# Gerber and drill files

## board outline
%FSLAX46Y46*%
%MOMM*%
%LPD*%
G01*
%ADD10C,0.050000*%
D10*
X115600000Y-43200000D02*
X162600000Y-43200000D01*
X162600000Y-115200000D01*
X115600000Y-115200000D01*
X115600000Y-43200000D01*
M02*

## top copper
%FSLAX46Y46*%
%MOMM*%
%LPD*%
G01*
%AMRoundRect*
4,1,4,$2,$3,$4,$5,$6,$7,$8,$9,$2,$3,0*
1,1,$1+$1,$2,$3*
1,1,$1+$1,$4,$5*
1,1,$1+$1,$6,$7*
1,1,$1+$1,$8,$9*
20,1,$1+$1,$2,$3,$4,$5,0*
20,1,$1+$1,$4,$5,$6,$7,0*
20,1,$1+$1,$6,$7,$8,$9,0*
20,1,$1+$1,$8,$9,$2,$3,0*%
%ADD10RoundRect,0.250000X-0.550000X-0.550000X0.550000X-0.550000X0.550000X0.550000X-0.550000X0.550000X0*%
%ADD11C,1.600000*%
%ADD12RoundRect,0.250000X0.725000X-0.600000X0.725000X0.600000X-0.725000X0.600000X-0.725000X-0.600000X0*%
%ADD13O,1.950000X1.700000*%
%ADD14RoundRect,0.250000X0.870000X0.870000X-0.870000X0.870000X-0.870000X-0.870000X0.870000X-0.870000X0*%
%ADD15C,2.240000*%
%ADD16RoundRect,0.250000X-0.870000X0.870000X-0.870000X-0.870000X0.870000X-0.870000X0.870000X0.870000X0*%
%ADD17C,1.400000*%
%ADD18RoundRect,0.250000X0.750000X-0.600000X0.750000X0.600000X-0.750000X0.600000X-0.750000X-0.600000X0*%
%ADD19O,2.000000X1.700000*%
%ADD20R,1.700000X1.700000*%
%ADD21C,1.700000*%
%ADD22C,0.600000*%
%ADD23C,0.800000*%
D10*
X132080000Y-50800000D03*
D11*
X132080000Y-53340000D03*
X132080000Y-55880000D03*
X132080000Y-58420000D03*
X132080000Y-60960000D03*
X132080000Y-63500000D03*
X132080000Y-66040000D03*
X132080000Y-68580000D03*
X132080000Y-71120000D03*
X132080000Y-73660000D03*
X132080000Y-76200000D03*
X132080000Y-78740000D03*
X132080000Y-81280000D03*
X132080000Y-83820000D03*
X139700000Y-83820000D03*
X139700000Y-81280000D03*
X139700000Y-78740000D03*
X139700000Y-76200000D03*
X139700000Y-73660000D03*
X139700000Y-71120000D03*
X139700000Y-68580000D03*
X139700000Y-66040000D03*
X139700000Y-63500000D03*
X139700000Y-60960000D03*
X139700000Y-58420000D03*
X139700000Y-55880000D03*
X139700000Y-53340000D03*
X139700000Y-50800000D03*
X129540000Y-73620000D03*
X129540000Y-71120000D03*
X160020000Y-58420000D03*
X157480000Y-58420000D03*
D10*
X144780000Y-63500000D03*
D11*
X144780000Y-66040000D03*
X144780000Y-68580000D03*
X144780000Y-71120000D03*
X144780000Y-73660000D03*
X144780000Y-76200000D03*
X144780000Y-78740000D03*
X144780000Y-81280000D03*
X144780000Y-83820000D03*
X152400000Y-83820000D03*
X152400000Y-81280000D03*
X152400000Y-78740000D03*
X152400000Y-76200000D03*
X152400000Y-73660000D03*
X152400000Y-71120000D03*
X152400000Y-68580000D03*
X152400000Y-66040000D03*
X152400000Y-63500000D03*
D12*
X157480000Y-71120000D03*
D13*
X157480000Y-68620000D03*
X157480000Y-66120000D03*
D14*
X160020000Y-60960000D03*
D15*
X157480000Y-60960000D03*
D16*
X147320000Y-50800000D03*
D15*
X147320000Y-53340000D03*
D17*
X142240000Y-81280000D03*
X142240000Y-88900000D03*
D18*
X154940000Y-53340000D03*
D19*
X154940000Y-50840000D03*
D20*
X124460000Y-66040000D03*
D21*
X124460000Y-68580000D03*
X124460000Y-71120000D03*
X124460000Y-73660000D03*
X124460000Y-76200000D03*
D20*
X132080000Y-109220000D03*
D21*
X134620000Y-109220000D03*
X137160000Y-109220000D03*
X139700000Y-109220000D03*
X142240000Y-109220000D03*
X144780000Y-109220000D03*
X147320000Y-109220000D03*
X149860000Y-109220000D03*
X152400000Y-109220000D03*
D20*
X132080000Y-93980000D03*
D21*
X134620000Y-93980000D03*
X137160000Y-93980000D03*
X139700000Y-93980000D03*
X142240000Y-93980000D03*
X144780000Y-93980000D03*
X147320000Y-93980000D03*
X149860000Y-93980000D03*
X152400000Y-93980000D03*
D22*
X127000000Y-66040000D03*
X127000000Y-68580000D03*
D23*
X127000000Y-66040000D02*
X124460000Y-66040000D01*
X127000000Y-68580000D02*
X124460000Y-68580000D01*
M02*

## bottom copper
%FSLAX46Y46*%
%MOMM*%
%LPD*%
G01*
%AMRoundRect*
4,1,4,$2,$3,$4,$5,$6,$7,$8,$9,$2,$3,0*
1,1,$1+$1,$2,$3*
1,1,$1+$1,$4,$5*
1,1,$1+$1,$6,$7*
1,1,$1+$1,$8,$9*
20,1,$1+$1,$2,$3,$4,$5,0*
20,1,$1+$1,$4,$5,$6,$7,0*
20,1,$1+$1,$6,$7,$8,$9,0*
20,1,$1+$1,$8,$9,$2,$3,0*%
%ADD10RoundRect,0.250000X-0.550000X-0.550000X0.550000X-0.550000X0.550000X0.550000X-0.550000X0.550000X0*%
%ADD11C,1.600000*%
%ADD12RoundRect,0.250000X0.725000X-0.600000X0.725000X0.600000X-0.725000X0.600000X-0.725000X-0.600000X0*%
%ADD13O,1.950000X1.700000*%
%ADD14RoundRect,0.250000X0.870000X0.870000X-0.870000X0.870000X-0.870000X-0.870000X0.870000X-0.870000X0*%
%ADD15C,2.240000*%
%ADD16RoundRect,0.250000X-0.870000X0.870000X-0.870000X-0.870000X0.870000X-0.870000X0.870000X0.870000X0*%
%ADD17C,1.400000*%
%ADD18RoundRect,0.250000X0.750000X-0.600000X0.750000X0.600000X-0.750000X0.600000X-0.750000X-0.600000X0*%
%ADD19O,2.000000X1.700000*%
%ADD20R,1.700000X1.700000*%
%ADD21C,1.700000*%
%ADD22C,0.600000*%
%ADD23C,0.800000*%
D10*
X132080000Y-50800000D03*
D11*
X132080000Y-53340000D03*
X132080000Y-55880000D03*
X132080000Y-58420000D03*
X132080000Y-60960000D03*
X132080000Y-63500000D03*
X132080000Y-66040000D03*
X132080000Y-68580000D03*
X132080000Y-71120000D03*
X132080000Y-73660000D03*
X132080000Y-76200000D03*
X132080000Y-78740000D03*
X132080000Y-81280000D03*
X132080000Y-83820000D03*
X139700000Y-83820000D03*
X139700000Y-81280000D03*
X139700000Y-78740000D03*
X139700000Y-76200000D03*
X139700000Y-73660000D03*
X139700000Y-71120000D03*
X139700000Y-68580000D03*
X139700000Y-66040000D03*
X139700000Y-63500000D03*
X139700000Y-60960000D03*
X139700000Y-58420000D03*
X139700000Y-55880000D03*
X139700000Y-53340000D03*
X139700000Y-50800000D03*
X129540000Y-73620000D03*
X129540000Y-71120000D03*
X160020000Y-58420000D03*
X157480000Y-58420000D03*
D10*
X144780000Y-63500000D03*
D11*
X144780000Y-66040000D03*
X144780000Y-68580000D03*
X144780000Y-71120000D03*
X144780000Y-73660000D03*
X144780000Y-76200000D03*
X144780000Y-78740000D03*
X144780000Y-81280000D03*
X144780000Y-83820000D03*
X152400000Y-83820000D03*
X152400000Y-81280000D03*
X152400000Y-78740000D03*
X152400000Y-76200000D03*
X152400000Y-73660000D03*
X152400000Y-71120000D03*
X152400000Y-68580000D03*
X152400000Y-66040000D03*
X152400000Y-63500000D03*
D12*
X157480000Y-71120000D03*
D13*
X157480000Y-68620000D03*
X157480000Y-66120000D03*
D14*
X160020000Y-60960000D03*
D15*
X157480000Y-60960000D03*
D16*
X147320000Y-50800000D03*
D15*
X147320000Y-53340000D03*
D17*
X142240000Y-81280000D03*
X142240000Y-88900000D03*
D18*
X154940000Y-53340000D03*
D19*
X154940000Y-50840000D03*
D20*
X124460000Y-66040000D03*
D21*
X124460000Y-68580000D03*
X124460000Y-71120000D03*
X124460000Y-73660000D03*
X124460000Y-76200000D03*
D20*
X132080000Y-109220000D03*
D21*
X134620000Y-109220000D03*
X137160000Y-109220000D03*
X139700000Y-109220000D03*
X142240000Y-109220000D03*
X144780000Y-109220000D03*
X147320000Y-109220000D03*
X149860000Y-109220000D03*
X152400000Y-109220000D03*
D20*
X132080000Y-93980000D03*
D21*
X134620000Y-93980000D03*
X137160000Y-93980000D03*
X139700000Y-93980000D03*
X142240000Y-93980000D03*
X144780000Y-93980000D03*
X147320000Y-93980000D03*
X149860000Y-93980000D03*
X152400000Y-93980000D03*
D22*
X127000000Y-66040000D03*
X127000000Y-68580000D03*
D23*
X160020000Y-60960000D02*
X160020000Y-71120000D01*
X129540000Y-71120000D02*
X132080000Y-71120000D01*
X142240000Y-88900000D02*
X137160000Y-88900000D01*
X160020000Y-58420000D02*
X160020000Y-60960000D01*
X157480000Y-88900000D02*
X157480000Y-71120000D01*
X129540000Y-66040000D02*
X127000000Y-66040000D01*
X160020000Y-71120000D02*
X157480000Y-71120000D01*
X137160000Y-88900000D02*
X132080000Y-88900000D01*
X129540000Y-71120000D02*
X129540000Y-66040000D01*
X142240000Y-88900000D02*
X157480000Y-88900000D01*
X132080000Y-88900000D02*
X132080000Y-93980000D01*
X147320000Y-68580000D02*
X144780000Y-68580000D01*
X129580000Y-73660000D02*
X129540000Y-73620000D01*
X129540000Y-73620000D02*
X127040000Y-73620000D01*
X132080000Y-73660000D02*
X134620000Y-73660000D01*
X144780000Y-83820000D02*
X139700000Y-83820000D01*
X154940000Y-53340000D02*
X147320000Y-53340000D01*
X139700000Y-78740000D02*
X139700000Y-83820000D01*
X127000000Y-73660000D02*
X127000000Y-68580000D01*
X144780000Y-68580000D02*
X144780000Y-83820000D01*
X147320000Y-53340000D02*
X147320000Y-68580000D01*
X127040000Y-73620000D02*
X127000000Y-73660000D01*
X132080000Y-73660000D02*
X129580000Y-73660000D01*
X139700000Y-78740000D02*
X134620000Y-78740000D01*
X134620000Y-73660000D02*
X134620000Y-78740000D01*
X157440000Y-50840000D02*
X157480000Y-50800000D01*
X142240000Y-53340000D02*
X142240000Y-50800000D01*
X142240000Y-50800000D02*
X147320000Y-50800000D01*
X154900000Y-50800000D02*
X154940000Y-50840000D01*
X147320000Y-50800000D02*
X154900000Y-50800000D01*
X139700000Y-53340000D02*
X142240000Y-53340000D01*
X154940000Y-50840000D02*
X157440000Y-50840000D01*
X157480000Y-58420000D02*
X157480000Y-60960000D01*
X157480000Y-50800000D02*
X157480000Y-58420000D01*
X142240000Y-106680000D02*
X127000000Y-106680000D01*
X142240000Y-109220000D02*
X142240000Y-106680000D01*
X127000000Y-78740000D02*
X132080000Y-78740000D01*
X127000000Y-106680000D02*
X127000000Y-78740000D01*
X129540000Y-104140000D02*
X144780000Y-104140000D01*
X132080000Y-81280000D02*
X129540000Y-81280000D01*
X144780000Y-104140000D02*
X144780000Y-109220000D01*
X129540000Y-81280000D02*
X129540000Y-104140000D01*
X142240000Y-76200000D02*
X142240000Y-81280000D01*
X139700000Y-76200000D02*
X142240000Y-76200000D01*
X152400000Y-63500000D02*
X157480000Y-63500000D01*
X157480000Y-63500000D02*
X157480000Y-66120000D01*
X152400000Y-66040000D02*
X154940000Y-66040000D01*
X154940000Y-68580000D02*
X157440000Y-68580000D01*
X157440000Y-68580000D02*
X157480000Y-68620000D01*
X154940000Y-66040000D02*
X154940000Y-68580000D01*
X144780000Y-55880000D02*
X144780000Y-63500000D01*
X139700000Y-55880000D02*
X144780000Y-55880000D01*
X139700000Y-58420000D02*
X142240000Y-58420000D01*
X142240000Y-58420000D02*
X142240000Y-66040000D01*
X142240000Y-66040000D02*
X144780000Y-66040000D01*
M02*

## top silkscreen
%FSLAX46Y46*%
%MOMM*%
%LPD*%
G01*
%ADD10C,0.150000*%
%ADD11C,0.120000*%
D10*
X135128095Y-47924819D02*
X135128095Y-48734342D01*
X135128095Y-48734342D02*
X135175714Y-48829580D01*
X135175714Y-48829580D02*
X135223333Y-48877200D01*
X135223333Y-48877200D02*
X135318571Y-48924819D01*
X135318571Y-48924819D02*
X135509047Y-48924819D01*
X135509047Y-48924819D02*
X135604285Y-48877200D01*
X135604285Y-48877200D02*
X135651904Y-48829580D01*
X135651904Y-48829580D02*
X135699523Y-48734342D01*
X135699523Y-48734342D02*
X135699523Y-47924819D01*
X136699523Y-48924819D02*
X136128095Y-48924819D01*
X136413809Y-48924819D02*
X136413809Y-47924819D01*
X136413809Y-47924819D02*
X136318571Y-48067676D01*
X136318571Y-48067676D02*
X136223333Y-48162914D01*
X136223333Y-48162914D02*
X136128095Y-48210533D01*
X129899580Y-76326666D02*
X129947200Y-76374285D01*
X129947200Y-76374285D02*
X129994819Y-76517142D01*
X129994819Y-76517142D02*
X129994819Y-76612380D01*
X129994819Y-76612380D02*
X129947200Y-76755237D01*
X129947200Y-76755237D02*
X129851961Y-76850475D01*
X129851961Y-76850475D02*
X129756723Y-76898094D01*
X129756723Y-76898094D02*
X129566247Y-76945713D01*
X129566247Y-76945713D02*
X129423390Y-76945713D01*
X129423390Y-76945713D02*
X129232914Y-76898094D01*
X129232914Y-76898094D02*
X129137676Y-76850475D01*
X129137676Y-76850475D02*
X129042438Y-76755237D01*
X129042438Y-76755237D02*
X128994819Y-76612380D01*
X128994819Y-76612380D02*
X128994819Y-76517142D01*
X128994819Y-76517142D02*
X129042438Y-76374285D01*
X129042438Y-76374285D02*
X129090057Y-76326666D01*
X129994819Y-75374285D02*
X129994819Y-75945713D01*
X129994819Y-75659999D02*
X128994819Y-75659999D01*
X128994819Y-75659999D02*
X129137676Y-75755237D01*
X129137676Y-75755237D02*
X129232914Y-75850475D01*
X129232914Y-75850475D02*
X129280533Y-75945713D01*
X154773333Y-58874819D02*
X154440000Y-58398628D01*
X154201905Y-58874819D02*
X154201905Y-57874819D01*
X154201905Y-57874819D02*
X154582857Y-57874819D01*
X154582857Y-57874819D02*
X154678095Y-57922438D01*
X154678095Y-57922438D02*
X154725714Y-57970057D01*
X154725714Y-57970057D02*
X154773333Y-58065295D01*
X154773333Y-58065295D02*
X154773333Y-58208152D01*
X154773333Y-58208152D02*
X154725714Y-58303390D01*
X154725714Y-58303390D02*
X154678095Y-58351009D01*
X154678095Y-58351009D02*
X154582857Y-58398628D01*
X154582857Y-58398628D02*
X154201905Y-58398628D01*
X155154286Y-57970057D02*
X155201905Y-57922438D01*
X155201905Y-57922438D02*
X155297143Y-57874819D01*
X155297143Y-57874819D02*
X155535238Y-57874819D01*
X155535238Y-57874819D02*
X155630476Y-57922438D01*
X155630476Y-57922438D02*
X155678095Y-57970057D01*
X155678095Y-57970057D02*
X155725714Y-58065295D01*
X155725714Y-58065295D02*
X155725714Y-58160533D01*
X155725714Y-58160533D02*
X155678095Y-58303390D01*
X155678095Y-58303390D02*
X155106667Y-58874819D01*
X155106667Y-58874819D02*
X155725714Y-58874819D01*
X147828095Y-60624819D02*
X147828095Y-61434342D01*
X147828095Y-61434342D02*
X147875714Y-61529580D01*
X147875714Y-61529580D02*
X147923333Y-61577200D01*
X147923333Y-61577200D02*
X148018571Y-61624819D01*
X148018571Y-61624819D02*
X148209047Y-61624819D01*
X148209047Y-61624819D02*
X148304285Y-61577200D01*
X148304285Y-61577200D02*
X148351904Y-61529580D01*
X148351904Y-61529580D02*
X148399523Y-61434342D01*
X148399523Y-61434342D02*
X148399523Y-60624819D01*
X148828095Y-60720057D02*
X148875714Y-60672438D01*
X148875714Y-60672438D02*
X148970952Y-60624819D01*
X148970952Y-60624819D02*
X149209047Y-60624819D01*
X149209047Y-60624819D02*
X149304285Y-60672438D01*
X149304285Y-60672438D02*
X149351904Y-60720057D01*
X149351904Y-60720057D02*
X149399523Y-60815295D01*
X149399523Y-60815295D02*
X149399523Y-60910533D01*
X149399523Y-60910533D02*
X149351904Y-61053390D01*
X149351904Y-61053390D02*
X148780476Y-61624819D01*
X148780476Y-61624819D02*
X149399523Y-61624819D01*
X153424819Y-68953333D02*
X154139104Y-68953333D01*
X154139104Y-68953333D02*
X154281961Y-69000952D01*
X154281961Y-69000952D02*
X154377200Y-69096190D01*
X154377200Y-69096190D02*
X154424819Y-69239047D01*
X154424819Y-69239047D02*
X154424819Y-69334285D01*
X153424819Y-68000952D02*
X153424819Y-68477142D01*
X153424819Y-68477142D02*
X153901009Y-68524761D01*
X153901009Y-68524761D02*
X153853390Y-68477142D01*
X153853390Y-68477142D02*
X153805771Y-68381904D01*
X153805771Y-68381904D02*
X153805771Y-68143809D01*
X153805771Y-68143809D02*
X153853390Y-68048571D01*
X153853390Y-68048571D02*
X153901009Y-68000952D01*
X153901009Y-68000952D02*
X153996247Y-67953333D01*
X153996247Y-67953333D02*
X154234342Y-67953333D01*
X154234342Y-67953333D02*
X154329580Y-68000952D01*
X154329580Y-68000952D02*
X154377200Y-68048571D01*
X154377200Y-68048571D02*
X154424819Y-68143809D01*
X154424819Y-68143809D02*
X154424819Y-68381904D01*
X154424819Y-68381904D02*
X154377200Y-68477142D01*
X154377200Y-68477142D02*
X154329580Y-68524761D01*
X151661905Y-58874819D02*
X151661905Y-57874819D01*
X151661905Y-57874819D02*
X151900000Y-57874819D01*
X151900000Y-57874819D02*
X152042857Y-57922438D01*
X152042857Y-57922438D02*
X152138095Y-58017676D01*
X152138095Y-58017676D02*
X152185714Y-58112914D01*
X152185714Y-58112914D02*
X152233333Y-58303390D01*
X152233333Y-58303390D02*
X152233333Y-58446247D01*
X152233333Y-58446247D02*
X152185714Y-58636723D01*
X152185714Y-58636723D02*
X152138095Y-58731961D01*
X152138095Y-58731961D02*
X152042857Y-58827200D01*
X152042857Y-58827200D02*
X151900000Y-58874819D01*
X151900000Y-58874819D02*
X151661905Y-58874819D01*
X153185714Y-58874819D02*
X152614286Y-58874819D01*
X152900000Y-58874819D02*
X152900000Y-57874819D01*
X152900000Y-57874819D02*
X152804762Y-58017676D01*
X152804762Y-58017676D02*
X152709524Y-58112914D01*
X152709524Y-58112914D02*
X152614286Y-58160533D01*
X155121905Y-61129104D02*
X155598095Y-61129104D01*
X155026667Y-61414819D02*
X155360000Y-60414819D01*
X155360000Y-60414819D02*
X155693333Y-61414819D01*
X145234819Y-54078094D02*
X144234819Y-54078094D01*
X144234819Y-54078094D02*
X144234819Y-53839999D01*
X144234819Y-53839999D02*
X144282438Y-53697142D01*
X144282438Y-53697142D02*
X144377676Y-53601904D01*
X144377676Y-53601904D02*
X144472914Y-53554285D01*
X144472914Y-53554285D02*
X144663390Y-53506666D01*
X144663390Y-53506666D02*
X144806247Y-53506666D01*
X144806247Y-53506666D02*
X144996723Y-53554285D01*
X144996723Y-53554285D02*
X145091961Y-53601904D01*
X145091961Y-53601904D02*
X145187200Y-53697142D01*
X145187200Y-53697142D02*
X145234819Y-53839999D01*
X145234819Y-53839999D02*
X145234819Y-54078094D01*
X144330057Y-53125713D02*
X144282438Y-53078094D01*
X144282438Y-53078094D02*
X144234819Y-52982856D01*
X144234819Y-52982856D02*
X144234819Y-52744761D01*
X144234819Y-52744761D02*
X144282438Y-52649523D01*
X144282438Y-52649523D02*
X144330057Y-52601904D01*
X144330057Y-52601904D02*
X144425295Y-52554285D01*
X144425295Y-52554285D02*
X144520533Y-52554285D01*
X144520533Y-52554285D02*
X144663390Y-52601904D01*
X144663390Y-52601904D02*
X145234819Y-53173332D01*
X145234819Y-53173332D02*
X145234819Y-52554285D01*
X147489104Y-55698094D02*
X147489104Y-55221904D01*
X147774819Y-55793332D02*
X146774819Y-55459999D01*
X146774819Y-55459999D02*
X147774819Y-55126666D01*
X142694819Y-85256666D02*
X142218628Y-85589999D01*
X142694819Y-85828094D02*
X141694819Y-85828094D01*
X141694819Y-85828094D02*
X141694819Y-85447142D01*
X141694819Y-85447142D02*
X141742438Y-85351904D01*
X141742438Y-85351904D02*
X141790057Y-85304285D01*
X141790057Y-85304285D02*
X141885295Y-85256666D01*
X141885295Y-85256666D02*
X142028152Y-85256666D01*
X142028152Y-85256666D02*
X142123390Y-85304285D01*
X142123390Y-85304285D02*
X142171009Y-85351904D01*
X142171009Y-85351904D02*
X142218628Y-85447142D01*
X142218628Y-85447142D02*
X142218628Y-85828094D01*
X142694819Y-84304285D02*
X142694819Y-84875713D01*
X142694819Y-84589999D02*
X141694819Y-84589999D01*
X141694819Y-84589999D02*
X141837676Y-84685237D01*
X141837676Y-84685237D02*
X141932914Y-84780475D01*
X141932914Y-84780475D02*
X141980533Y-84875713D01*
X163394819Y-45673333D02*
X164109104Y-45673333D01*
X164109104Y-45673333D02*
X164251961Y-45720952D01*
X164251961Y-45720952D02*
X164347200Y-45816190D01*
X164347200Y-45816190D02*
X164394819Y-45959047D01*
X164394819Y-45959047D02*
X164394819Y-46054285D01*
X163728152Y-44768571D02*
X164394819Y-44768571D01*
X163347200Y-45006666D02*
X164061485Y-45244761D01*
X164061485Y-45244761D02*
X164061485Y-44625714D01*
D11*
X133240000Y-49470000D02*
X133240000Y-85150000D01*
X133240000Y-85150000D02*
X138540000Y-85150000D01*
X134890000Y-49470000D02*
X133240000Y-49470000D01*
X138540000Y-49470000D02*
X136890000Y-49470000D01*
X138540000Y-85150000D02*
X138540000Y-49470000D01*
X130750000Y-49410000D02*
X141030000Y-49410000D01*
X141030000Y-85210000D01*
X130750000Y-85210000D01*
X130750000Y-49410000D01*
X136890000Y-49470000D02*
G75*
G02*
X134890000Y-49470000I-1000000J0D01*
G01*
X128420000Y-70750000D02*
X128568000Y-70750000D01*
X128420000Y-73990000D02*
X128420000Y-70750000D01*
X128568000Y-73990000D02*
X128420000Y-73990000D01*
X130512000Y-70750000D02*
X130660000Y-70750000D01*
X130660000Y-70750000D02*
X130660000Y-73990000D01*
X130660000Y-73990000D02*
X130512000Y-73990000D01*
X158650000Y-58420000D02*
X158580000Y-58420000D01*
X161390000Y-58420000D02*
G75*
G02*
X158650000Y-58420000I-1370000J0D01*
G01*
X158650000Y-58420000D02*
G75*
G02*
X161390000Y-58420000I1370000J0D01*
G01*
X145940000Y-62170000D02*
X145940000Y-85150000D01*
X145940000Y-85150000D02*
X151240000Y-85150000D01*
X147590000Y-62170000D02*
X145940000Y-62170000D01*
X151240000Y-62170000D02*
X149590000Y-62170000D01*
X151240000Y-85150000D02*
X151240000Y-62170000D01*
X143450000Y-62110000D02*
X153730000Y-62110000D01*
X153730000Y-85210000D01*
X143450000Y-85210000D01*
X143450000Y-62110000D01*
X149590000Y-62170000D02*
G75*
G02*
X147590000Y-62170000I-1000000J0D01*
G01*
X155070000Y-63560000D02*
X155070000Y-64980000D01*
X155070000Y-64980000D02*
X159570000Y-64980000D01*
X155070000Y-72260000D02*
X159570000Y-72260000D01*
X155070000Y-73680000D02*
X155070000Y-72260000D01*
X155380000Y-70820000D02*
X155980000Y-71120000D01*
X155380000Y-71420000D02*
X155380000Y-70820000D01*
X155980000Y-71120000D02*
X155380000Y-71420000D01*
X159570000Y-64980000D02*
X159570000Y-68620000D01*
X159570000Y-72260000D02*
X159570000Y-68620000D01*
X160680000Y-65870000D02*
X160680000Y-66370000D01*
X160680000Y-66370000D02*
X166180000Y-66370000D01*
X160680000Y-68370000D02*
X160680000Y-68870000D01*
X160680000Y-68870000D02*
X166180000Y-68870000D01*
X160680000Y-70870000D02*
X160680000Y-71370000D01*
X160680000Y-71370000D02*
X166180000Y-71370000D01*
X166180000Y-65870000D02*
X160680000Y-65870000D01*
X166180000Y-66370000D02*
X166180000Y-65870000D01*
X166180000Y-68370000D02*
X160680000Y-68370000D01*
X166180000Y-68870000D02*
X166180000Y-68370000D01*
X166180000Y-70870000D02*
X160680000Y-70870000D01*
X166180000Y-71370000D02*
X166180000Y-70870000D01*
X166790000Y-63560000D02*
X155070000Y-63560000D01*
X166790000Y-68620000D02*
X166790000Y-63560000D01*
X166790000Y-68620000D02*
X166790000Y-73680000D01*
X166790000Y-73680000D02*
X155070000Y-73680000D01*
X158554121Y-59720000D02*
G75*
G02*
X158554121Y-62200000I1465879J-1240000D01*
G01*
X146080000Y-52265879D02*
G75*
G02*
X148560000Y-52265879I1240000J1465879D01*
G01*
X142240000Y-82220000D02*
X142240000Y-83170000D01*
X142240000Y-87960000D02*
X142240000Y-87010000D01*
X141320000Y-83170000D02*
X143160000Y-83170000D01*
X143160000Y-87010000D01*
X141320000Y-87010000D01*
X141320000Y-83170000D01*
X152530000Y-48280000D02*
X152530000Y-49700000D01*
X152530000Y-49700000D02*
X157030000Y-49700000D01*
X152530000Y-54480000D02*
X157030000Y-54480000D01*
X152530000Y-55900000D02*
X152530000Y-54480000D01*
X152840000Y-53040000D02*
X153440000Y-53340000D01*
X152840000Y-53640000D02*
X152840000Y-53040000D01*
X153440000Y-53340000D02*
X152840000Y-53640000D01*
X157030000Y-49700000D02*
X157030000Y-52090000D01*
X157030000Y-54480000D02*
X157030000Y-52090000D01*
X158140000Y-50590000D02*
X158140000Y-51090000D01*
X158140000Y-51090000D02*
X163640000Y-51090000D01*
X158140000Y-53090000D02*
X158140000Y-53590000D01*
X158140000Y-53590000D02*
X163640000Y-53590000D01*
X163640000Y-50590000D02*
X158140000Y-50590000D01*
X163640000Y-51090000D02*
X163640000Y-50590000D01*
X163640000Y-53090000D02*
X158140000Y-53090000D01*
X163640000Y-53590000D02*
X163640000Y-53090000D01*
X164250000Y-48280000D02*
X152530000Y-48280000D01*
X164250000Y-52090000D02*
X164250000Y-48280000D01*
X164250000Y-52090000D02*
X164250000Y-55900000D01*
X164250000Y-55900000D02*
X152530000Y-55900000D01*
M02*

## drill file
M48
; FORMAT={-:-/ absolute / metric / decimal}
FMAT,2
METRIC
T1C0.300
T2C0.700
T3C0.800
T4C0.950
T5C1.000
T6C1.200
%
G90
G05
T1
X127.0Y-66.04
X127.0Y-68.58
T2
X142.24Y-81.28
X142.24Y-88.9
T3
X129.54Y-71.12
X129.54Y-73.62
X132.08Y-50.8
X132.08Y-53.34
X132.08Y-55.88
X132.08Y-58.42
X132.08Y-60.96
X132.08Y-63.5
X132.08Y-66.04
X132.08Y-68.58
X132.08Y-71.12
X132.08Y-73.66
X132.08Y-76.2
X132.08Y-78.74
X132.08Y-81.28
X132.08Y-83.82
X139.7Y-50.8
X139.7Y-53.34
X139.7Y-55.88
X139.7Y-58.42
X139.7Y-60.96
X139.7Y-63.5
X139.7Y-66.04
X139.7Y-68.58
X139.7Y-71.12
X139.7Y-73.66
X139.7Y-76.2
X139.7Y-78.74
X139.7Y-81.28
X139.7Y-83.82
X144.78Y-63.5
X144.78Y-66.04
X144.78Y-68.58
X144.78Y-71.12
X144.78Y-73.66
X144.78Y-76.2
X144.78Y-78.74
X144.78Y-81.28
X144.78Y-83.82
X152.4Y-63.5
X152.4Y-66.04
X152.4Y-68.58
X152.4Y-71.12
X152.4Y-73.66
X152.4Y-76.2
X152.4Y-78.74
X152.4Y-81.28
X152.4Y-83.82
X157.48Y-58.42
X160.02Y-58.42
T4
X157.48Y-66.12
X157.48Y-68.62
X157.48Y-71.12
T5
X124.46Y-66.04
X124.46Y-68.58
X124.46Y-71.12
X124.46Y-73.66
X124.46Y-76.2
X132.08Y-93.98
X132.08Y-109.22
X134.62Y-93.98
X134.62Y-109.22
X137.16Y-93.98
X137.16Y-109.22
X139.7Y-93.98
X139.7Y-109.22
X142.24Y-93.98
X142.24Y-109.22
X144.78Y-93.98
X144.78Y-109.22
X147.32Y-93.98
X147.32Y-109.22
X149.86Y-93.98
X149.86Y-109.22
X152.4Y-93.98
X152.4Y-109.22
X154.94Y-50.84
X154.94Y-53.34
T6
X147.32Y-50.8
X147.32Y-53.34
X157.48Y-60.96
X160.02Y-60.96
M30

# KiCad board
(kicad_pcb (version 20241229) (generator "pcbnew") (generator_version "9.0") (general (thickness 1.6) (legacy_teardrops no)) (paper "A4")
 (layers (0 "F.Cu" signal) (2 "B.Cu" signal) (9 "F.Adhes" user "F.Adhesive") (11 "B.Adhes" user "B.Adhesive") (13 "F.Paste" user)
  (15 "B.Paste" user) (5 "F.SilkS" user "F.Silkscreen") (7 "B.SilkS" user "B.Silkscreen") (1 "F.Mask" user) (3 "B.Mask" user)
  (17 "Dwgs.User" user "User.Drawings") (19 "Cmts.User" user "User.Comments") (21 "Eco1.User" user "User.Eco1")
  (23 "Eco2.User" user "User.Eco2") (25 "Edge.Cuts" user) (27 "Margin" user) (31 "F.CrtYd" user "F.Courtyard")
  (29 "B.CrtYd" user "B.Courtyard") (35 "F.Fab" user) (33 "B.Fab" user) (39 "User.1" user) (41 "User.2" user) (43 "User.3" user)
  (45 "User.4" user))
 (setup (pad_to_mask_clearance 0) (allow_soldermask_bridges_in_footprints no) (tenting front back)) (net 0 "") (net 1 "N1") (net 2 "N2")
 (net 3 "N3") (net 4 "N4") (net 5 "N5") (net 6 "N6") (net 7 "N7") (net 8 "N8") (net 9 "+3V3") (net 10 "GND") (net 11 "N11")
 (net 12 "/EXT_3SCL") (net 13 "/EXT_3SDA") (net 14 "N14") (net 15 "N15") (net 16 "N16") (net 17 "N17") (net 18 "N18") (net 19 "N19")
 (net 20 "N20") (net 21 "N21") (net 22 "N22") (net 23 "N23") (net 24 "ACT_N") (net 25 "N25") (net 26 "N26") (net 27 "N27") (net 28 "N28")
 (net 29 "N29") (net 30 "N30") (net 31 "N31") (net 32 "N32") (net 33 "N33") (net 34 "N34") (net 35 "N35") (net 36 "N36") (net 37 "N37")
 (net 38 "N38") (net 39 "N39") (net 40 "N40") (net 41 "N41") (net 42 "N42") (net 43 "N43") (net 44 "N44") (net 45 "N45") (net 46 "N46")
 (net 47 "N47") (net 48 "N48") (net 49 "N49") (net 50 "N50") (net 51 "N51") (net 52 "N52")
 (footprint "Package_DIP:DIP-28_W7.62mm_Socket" (layer "F.Cu") (at 132.08 50.8)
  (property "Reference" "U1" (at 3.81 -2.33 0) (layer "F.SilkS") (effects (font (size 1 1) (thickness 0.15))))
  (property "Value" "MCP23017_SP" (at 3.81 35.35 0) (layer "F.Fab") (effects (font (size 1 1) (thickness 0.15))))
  (fp_line (start 1.16 -1.33) (end 1.16 34.35) (stroke (width 0.12) (type solid)) (layer "F.SilkS"))
  (fp_line (start 1.16 34.35) (end 6.46 34.35) (stroke (width 0.12) (type solid)) (layer "F.SilkS"))
  (fp_line (start 2.81 -1.33) (end 1.16 -1.33) (stroke (width 0.12) (type solid)) (layer "F.SilkS"))
  (fp_line (start 6.46 -1.33) (end 4.81 -1.33) (stroke (width 0.12) (type solid)) (layer "F.SilkS"))
  (fp_line (start 6.46 34.35) (end 6.46 -1.33) (stroke (width 0.12) (type solid)) (layer "F.SilkS"))
  (fp_rect (start -1.33 -1.39) (end 8.95 34.41) (stroke (width 0.12) (type solid)) (fill no) (layer "F.SilkS"))
  (fp_arc (start 4.81 -1.33) (mid 3.81 -0.33) (end 2.81 -1.33) (stroke (width 0.12) (type solid)) (layer "F.SilkS"))
  (pad "1" thru_hole roundrect (at 0 0) (size 1.6 1.6) (drill 0.8) (layers "*.Cu" "*.Mask") (remove_unused_layers no)
   (roundrect_rratio 0.15625) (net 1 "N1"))
  (pad "2" thru_hole circle (at 0 2.54) (size 1.6 1.6) (drill 0.8) (layers "*.Cu" "*.Mask") (remove_unused_layers no) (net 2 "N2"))
  (pad "3" thru_hole circle (at 0 5.08) (size 1.6 1.6) (drill 0.8) (layers "*.Cu" "*.Mask") (remove_unused_layers no) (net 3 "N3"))
  (pad "4" thru_hole circle (at 0 7.62) (size 1.6 1.6) (drill 0.8) (layers "*.Cu" "*.Mask") (remove_unused_layers no) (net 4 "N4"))
  (pad "5" thru_hole circle (at 0 10.16) (size 1.6 1.6) (drill 0.8) (layers "*.Cu" "*.Mask") (remove_unused_layers no) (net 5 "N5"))
  (pad "6" thru_hole circle (at 0 12.7) (size 1.6 1.6) (drill 0.8) (layers "*.Cu" "*.Mask") (remove_unused_layers no) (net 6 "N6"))
  (pad "7" thru_hole circle (at 0 15.24) (size 1.6 1.6) (drill 0.8) (layers "*.Cu" "*.Mask") (remove_unused_layers no) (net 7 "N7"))
  (pad "8" thru_hole circle (at 0 17.78) (size 1.6 1.6) (drill 0.8) (layers "*.Cu" "*.Mask") (remove_unused_layers no) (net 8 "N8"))
  (pad "9" thru_hole circle (at 0 20.32) (size 1.6 1.6) (drill 0.8) (layers "*.Cu" "*.Mask") (remove_unused_layers no) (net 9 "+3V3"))
  (pad "10" thru_hole circle (at 0 22.86) (size 1.6 1.6) (drill 0.8) (layers "*.Cu" "*.Mask") (remove_unused_layers no) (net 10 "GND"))
  (pad "11" thru_hole circle (at 0 25.4) (size 1.6 1.6) (drill 0.8) (layers "*.Cu" "*.Mask") (remove_unused_layers no) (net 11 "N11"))
  (pad "12" thru_hole circle (at 0 27.94) (size 1.6 1.6) (drill 0.8) (layers "*.Cu" "*.Mask") (remove_unused_layers no) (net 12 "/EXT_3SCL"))
  (pad "13" thru_hole circle (at 0 30.48) (size 1.6 1.6) (drill 0.8) (layers "*.Cu" "*.Mask") (remove_unused_layers no) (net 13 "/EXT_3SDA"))
  (pad "14" thru_hole circle (at 0 33.02) (size 1.6 1.6) (drill 0.8) (layers "*.Cu" "*.Mask") (remove_unused_layers no) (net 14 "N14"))
  (pad "15" thru_hole circle (at 7.62 33.02) (size 1.6 1.6) (drill 0.8) (layers "*.Cu" "*.Mask") (remove_unused_layers no) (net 10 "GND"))
  (pad "16" thru_hole circle (at 7.62 30.48) (size 1.6 1.6) (drill 0.8) (layers "*.Cu" "*.Mask") (remove_unused_layers no) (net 10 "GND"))
  (pad "17" thru_hole circle (at 7.62 27.94) (size 1.6 1.6) (drill 0.8) (layers "*.Cu" "*.Mask") (remove_unused_layers no) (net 10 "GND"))
  (pad "18" thru_hole circle (at 7.62 25.4) (size 1.6 1.6) (drill 0.8) (layers "*.Cu" "*.Mask") (remove_unused_layers no) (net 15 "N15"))
  (pad "19" thru_hole circle (at 7.62 22.86) (size 1.6 1.6) (drill 0.8) (layers "*.Cu" "*.Mask") (remove_unused_layers no) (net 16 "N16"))
  (pad "20" thru_hole circle (at 7.62 20.32) (size 1.6 1.6) (drill 0.8) (layers "*.Cu" "*.Mask") (remove_unused_layers no) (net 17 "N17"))
  (pad "21" thru_hole circle (at 7.62 17.78) (size 1.6 1.6) (drill 0.8) (layers "*.Cu" "*.Mask") (remove_unused_layers no) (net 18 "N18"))
  (pad "22" thru_hole circle (at 7.62 15.24) (size 1.6 1.6) (drill 0.8) (layers "*.Cu" "*.Mask") (remove_unused_layers no) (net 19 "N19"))
  (pad "23" thru_hole circle (at 7.62 12.7) (size 1.6 1.6) (drill 0.8) (layers "*.Cu" "*.Mask") (remove_unused_layers no) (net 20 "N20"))
  (pad "24" thru_hole circle (at 7.62 10.16) (size 1.6 1.6) (drill 0.8) (layers "*.Cu" "*.Mask") (remove_unused_layers no) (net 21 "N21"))
  (pad "25" thru_hole circle (at 7.62 7.62) (size 1.6 1.6) (drill 0.8) (layers "*.Cu" "*.Mask") (remove_unused_layers no) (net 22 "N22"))
  (pad "26" thru_hole circle (at 7.62 5.08) (size 1.6 1.6) (drill 0.8) (layers "*.Cu" "*.Mask") (remove_unused_layers no) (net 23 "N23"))
  (pad "27" thru_hole circle (at 7.62 2.54) (size 1.6 1.6) (drill 0.8) (layers "*.Cu" "*.Mask") (remove_unused_layers no) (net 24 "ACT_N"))
  (pad "28" thru_hole circle (at 7.62 0) (size 1.6 1.6) (drill 0.8) (layers "*.Cu" "*.Mask") (remove_unused_layers no) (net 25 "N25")))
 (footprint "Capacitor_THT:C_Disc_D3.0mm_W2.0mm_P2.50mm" (layer "F.Cu") (at 129.54 73.62 90)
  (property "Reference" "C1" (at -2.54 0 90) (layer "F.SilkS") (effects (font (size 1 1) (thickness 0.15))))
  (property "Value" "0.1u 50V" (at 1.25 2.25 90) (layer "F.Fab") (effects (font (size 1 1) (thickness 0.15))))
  (fp_line (start 2.87 -1.12) (end 2.87 -0.972) (stroke (width 0.12) (type solid)) (layer "F.SilkS"))
  (fp_line (start -0.37 -1.12) (end 2.87 -1.12) (stroke (width 0.12) (type solid)) (layer "F.SilkS"))
  (fp_line (start -0.37 -0.972) (end -0.37 -1.12) (stroke (width 0.12) (type solid)) (layer "F.SilkS"))
  (fp_line (start 2.87 0.972) (end 2.87 1.12) (stroke (width 0.12) (type solid)) (layer "F.SilkS"))
  (fp_line (start 2.87 1.12) (end -0.37 1.12) (stroke (width 0.12) (type solid)) (layer "F.SilkS"))
  (fp_line (start -0.37 1.12) (end -0.37 0.972) (stroke (width 0.12) (type solid)) (layer "F.SilkS"))
  (pad "1" thru_hole circle (at 0 0 90) (size 1.6 1.6) (drill 0.8) (layers "*.Cu" "*.Mask") (remove_unused_layers no) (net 10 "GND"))
  (pad "2" thru_hole circle (at 2.5 0 90) (size 1.6 1.6) (drill 0.8) (layers "*.Cu" "*.Mask") (remove_unused_layers no) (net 9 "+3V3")))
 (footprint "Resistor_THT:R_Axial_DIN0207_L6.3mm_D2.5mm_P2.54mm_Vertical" (layer "F.Cu") (at 160.02 58.42 180)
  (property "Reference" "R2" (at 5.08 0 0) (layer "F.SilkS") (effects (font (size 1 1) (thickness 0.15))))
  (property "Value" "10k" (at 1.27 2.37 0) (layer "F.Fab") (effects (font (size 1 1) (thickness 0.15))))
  (fp_line (start 1.37 0) (end 1.44 0) (stroke (width 0.12) (type solid)) (layer "F.SilkS"))
  (fp_circle (center 0 0) (end 1.37 0) (stroke (width 0.12) (type solid)) (fill no) (layer "F.SilkS"))
  (pad "1" thru_hole circle (at 0 0 180) (size 1.6 1.6) (drill 0.8) (layers "*.Cu" "*.Mask") (remove_unused_layers no) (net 9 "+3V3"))
  (pad "2" thru_hole circle (at 2.54 0 180) (size 1.6 1.6) (drill 0.8) (layers "*.Cu" "*.Mask") (remove_unused_layers no) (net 24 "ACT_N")))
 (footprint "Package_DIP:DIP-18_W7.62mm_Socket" (layer "F.Cu") (at 144.78 63.5)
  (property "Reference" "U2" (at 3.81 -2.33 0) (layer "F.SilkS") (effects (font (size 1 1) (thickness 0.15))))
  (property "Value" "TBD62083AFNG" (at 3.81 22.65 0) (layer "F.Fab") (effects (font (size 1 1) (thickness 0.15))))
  (fp_line (start 1.16 -1.33) (end 1.16 21.65) (stroke (width 0.12) (type solid)) (layer "F.SilkS"))
  (fp_line (start 1.16 21.65) (end 6.46 21.65) (stroke (width 0.12) (type solid)) (layer "F.SilkS"))
  (fp_line (start 2.81 -1.33) (end 1.16 -1.33) (stroke (width 0.12) (type solid)) (layer "F.SilkS"))
  (fp_line (start 6.46 -1.33) (end 4.81 -1.33) (stroke (width 0.12) (type solid)) (layer "F.SilkS"))
  (fp_line (start 6.46 21.65) (end 6.46 -1.33) (stroke (width 0.12) (type solid)) (layer "F.SilkS"))
  (fp_rect (start -1.33 -1.39) (end 8.95 21.71) (stroke (width 0.12) (type solid)) (fill no) (layer "F.SilkS"))
  (fp_arc (start 4.81 -1.33) (mid 3.81 -0.33) (end 2.81 -1.33) (stroke (width 0.12) (type solid)) (layer "F.SilkS"))
  (pad "1" thru_hole roundrect (at 0 0) (size 1.6 1.6) (drill 0.8) (layers "*.Cu" "*.Mask") (remove_unused_layers no)
   (roundrect_rratio 0.15625) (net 23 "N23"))
  (pad "2" thru_hole circle (at 0 2.54) (size 1.6 1.6) (drill 0.8) (layers "*.Cu" "*.Mask") (remove_unused_layers no) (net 22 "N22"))
  (pad "3" thru_hole circle (at 0 5.08) (size 1.6 1.6) (drill 0.8) (layers "*.Cu" "*.Mask") (remove_unused_layers no) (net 10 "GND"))
  (pad "4" thru_hole circle (at 0 7.62) (size 1.6 1.6) (drill 0.8) (layers "*.Cu" "*.Mask") (remove_unused_layers no) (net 10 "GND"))
  (pad "5" thru_hole circle (at 0 10.16) (size 1.6 1.6) (drill 0.8) (layers "*.Cu" "*.Mask") (remove_unused_layers no) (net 10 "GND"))
  (pad "6" thru_hole circle (at 0 12.7) (size 1.6 1.6) (drill 0.8) (layers "*.Cu" "*.Mask") (remove_unused_layers no) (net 10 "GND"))
  (pad "7" thru_hole circle (at 0 15.24) (size 1.6 1.6) (drill 0.8) (layers "*.Cu" "*.Mask") (remove_unused_layers no) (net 10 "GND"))
  (pad "8" thru_hole circle (at 0 17.78) (size 1.6 1.6) (drill 0.8) (layers "*.Cu" "*.Mask") (remove_unused_layers no) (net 10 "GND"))
  (pad "9" thru_hole circle (at 0 20.32) (size 1.6 1.6) (drill 0.8) (layers "*.Cu" "*.Mask") (remove_unused_layers no) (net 10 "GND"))
  (pad "10" thru_hole circle (at 7.62 20.32) (size 1.6 1.6) (drill 0.8) (layers "*.Cu" "*.Mask") (remove_unused_layers no) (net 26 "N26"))
  (pad "11" thru_hole circle (at 7.62 17.78) (size 1.6 1.6) (drill 0.8) (layers "*.Cu" "*.Mask") (remove_unused_layers no) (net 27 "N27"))
  (pad "12" thru_hole circle (at 7.62 15.24) (size 1.6 1.6) (drill 0.8) (layers "*.Cu" "*.Mask") (remove_unused_layers no) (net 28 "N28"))
  (pad "13" thru_hole circle (at 7.62 12.7) (size 1.6 1.6) (drill 0.8) (layers "*.Cu" "*.Mask") (remove_unused_layers no) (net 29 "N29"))
  (pad "14" thru_hole circle (at 7.62 10.16) (size 1.6 1.6) (drill 0.8) (layers "*.Cu" "*.Mask") (remove_unused_layers no) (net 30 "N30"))
  (pad "15" thru_hole circle (at 7.62 7.62) (size 1.6 1.6) (drill 0.8) (layers "*.Cu" "*.Mask") (remove_unused_layers no) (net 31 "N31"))
  (pad "16" thru_hole circle (at 7.62 5.08) (size 1.6 1.6) (drill 0.8) (layers "*.Cu" "*.Mask") (remove_unused_layers no) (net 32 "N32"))
  (pad "17" thru_hole circle (at 7.62 2.54) (size 1.6 1.6) (drill 0.8) (layers "*.Cu" "*.Mask") (remove_unused_layers no) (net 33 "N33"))
  (pad "18" thru_hole circle (at 7.62 0) (size 1.6 1.6) (drill 0.8) (layers "*.Cu" "*.Mask") (remove_unused_layers no) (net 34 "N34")))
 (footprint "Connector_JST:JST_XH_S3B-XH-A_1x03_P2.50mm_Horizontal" (layer "F.Cu") (at 157.48 71.12 90)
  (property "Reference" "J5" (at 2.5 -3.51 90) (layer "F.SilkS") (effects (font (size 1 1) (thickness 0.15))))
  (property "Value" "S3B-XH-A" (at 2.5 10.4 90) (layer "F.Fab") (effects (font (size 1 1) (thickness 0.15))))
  (fp_line (start 7.56 -2.41) (end 6.14 -2.41) (stroke (width 0.12) (type solid)) (layer "F.SilkS"))
  (fp_line (start 6.14 -2.41) (end 6.14 2.09) (stroke (width 0.12) (type solid)) (layer "F.SilkS"))
  (fp_line (start -1.14 -2.41) (end -1.14 2.09) (stroke (width 0.12) (type solid)) (layer "F.SilkS"))
  (fp_line (start -2.56 -2.41) (end -1.14 -2.41) (stroke (width 0.12) (type solid)) (layer "F.SilkS"))
  (fp_line (start 0.3 -2.1) (end 0 -1.5) (stroke (width 0.12) (type solid)) (layer "F.SilkS"))
  (fp_line (start -0.3 -2.1) (end 0.3 -2.1) (stroke (width 0.12) (type solid)) (layer "F.SilkS"))
  (fp_line (start 0 -1.5) (end -0.3 -2.1) (stroke (width 0.12) (type solid)) (layer "F.SilkS"))
  (fp_line (start 6.14 2.09) (end 2.5 2.09) (stroke (width 0.12) (type solid)) (layer "F.SilkS"))
  (fp_line (start -1.14 2.09) (end 2.5 2.09) (stroke (width 0.12) (type solid)) (layer "F.SilkS"))
  (fp_line (start 5.25 3.2) (end 4.75 3.2) (stroke (width 0.12) (type solid)) (layer "F.SilkS"))
  (fp_line (start 4.75 3.2) (end 4.75 8.7) (stroke (width 0.12) (type solid)) (layer "F.SilkS"))
  (fp_line (start 2.75 3.2) (end 2.25 3.2) (stroke (width 0.12) (type solid)) (layer "F.SilkS"))
  (fp_line (start 2.25 3.2) (end 2.25 8.7) (stroke (width 0.12) (type solid)) (layer "F.SilkS"))
  (fp_line (start 0.25 3.2) (end -0.25 3.2) (stroke (width 0.12) (type solid)) (layer "F.SilkS"))
  (fp_line (start -0.25 3.2) (end -0.25 8.7) (stroke (width 0.12) (type solid)) (layer "F.SilkS"))
  (fp_line (start 5.25 8.7) (end 5.25 3.2) (stroke (width 0.12) (type solid)) (layer "F.SilkS"))
  (fp_line (start 4.75 8.7) (end 5.25 8.7) (stroke (width 0.12) (type solid)) (layer "F.SilkS"))
  (fp_line (start 2.75 8.7) (end 2.75 3.2) (stroke (width 0.12) (type solid)) (layer "F.SilkS"))
  (fp_line (start 2.25 8.7) (end 2.75 8.7) (stroke (width 0.12) (type solid)) (layer "F.SilkS"))
  (fp_line (start 0.25 8.7) (end 0.25 3.2) (stroke (width 0.12) (type solid)) (layer "F.SilkS"))
  (fp_line (start -0.25 8.7) (end 0.25 8.7) (stroke (width 0.12) (type solid)) (layer "F.SilkS"))
  (fp_line (start 7.56 9.31) (end 7.56 -2.41) (stroke (width 0.12) (type solid)) (layer "F.SilkS"))
  (fp_line (start 2.5 9.31) (end 7.56 9.31) (stroke (width 0.12) (type solid)) (layer "F.SilkS"))
  (fp_line (start 2.5 9.31) (end -2.56 9.31) (stroke (width 0.12) (type solid)) (layer "F.SilkS"))
  (fp_line (start -2.56 9.31) (end -2.56 -2.41) (stroke (width 0.12) (type solid)) (layer "F.SilkS"))
  (pad "1" thru_hole roundrect (at 0 0 90) (size 1.7 1.95) (drill 0.95) (layers "*.Cu" "*.Mask") (remove_unused_layers no)
   (roundrect_rratio 0.147059) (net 9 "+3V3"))
  (pad "2" thru_hole oval (at 2.5 0 90) (size 1.7 1.95) (drill 0.95) (layers "*.Cu" "*.Mask") (remove_unused_layers no) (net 33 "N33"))
  (pad "3" thru_hole oval (at 5 0 90) (size 1.7 1.95) (drill 0.95) (layers "*.Cu" "*.Mask") (remove_unused_layers no) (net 34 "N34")))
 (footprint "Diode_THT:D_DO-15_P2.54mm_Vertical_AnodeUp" (layer "F.Cu") (at 160.02 60.96 180)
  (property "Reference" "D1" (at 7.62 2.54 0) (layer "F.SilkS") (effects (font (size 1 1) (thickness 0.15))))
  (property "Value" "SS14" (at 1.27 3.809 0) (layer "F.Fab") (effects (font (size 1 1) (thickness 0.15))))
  (fp_arc (start 1.465879 1.24) (mid -1.92 0) (end 1.465879 -1.24) (stroke (width 0.12) (type solid)) (layer "F.SilkS"))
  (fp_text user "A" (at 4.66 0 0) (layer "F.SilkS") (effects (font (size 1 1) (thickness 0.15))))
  (pad "1" thru_hole roundrect (at 0 0 180) (size 2.24 2.24) (drill 1.2) (layers "*.Cu" "*.Mask") (remove_unused_layers no)
   (roundrect_rratio 0.111607) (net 9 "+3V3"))
  (pad "2" thru_hole circle (at 2.54 0 180) (size 2.24 2.24) (drill 1.2) (layers "*.Cu" "*.Mask") (remove_unused_layers no) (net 24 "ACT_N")))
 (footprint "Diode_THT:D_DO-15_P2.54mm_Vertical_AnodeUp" (layer "F.Cu") (at 147.32 50.8 -90)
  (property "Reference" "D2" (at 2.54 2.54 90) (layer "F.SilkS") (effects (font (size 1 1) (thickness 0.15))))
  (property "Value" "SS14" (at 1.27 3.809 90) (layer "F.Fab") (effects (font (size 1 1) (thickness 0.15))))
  (fp_arc (start 1.465879 1.24) (mid -1.92 0) (end 1.465879 -1.24) (stroke (width 0.12) (type solid)) (layer "F.SilkS"))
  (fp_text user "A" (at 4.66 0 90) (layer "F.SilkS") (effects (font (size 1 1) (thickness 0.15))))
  (pad "1" thru_hole roundrect (at 0 0 270) (size 2.24 2.24) (drill 1.2) (layers "*.Cu" "*.Mask") (remove_unused_layers no)
   (roundrect_rratio 0.111607) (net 24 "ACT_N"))
  (pad "2" thru_hole circle (at 2.54 0 270) (size 2.24 2.24) (drill 1.2) (layers "*.Cu" "*.Mask") (remove_unused_layers no) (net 10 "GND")))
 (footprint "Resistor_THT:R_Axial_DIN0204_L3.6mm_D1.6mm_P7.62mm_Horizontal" (layer "F.Cu") (at 142.24 81.28 -90)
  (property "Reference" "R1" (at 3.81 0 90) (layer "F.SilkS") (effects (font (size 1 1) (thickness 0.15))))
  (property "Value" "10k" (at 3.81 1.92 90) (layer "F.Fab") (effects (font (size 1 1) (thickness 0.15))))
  (fp_line (start 0.94 0) (end 1.89 0) (stroke (width 0.12) (type solid)) (layer "F.SilkS"))
  (fp_line (start 6.68 0) (end 5.73 0) (stroke (width 0.12) (type solid)) (layer "F.SilkS"))
  (fp_rect (start 1.89 -0.92) (end 5.73 0.92) (stroke (width 0.12) (type solid)) (fill no) (layer "F.SilkS"))
  (pad "1" thru_hole circle (at 0 0 270) (size 1.4 1.4) (drill 0.7) (layers "*.Cu" "*.Mask") (remove_unused_layers no) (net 15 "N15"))
  (pad "2" thru_hole circle (at 7.62 0 270) (size 1.4 1.4) (drill 0.7) (layers "*.Cu" "*.Mask") (remove_unused_layers no) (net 9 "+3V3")))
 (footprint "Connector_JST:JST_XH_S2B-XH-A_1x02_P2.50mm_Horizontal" (layer "F.Cu") (at 154.94 53.34 90)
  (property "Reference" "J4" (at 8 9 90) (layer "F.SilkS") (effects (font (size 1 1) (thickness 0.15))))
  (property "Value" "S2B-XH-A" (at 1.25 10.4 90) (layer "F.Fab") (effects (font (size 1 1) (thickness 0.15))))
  (fp_line (start 5.06 -2.41) (end 3.64 -2.41) (stroke (width 0.12) (type solid)) (layer "F.SilkS"))
  (fp_line (start 3.64 -2.41) (end 3.64 2.09) (stroke (width 0.12) (type solid)) (layer "F.SilkS"))
  (fp_line (start -1.14 -2.41) (end -1.14 2.09) (stroke (width 0.12) (type solid)) (layer "F.SilkS"))
  (fp_line (start -2.56 -2.41) (end -1.14 -2.41) (stroke (width 0.12) (type solid)) (layer "F.SilkS"))
  (fp_line (start 0.3 -2.1) (end 0 -1.5) (stroke (width 0.12) (type solid)) (layer "F.SilkS"))
  (fp_line (start -0.3 -2.1) (end 0.3 -2.1) (stroke (width 0.12) (type solid)) (layer "F.SilkS"))
  (fp_line (start 0 -1.5) (end -0.3 -2.1) (stroke (width 0.12) (type solid)) (layer "F.SilkS"))
  (fp_line (start 3.64 2.09) (end 1.25 2.09) (stroke (width 0.12) (type solid)) (layer "F.SilkS"))
  (fp_line (start -1.14 2.09) (end 1.25 2.09) (stroke (width 0.12) (type solid)) (layer "F.SilkS"))
  (fp_line (start 2.75 3.2) (end 2.25 3.2) (stroke (width 0.12) (type solid)) (layer "F.SilkS"))
  (fp_line (start 2.25 3.2) (end 2.25 8.7) (stroke (width 0.12) (type solid)) (layer "F.SilkS"))
  (fp_line (start 0.25 3.2) (end -0.25 3.2) (stroke (width 0.12) (type solid)) (layer "F.SilkS"))
  (fp_line (start -0.25 3.2) (end -0.25 8.7) (stroke (width 0.12) (type solid)) (layer "F.SilkS"))
  (fp_line (start 2.75 8.7) (end 2.75 3.2) (stroke (width 0.12) (type solid)) (layer "F.SilkS"))
  (fp_line (start 2.25 8.7) (end 2.75 8.7) (stroke (width 0.12) (type solid)) (layer "F.SilkS"))
  (fp_line (start 0.25 8.7) (end 0.25 3.2) (stroke (width 0.12) (type solid)) (layer "F.SilkS"))
  (fp_line (start -0.25 8.7) (end 0.25 8.7) (stroke (width 0.12) (type solid)) (layer "F.SilkS"))
  (fp_line (start 5.06 9.31) (end 5.06 -2.41) (stroke (width 0.12) (type solid)) (layer "F.SilkS"))
  (fp_line (start 1.25 9.31) (end 5.06 9.31) (stroke (width 0.12) (type solid)) (layer "F.SilkS"))
  (fp_line (start 1.25 9.31) (end -2.56 9.31) (stroke (width 0.12) (type solid)) (layer "F.SilkS"))
  (fp_line (start -2.56 9.31) (end -2.56 -2.41) (stroke (width 0.12) (type solid)) (layer "F.SilkS"))
  (pad "1" thru_hole roundrect (at 0 0 90) (size 1.7 2) (drill 1) (layers "*.Cu" "*.Mask") (remove_unused_layers no)
   (roundrect_rratio 0.147059) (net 10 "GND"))
  (pad "2" thru_hole oval (at 2.5 0 90) (size 1.7 2) (drill 1) (layers "*.Cu" "*.Mask") (remove_unused_layers no) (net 24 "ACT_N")))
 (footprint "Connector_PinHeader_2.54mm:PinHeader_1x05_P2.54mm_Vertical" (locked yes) (layer "B.Cu") (at 124.46 66.04 180)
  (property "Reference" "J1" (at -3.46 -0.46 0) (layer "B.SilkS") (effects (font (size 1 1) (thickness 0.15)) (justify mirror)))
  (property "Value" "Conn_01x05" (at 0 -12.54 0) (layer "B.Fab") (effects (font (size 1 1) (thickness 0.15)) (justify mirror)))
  (pad "1" thru_hole rect (at 0 0 180) (size 1.7 1.7) (drill 1) (layers "*.Cu" "*.Mask") (remove_unused_layers no) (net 9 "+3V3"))
  (pad "2" thru_hole circle (at 0 -2.54 180) (size 1.7 1.7) (drill 1) (layers "*.Cu" "*.Mask") (remove_unused_layers no) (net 10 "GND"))
  (pad "3" thru_hole circle (at 0 -5.08 180) (size 1.7 1.7) (drill 1) (layers "*.Cu" "*.Mask") (remove_unused_layers no) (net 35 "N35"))
  (pad "4" thru_hole circle (at 0 -7.62 180) (size 1.7 1.7) (drill 1) (layers "*.Cu" "*.Mask") (remove_unused_layers no) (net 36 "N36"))
  (pad "5" thru_hole circle (at 0 -10.16 180) (size 1.7 1.7) (drill 1) (layers "*.Cu" "*.Mask") (remove_unused_layers no) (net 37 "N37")))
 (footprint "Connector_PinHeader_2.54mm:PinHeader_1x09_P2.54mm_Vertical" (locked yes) (layer "B.Cu") (at 132.08 109.22 -90)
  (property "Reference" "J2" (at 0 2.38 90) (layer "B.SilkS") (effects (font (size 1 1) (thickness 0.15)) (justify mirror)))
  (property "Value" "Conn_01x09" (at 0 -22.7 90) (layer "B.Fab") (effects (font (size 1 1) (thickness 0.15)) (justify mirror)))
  (pad "1" thru_hole rect (at 0 0 270) (size 1.7 1.7) (drill 1) (layers "*.Cu" "*.Mask") (remove_unused_layers no) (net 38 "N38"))
  (pad "2" thru_hole circle (at 0 -2.54 270) (size 1.7 1.7) (drill 1) (layers "*.Cu" "*.Mask") (remove_unused_layers no) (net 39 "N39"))
  (pad "3" thru_hole circle (at 0 -5.08 270) (size 1.7 1.7) (drill 1) (layers "*.Cu" "*.Mask") (remove_unused_layers no) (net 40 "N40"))
  (pad "4" thru_hole circle (at 0 -7.62 270) (size 1.7 1.7) (drill 1) (layers "*.Cu" "*.Mask") (remove_unused_layers no) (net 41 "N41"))
  (pad "5" thru_hole circle (at 0 -10.16 270) (size 1.7 1.7) (drill 1) (layers "*.Cu" "*.Mask") (remove_unused_layers no)
   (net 12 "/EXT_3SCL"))
  (pad "6" thru_hole circle (at 0 -12.7 270) (size 1.7 1.7) (drill 1) (layers "*.Cu" "*.Mask") (remove_unused_layers no)
   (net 13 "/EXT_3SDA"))
  (pad "7" thru_hole circle (at 0 -15.24 270) (size 1.7 1.7) (drill 1) (layers "*.Cu" "*.Mask") (remove_unused_layers no) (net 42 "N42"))
  (pad "8" thru_hole circle (at 0 -17.78 270) (size 1.7 1.7) (drill 1) (layers "*.Cu" "*.Mask") (remove_unused_layers no) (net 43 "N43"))
  (pad "9" thru_hole circle (at 0 -20.32 270) (size 1.7 1.7) (drill 1) (layers "*.Cu" "*.Mask") (remove_unused_layers no) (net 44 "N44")))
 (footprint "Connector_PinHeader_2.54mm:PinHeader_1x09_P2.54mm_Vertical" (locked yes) (layer "B.Cu") (at 132.08 93.98 -90)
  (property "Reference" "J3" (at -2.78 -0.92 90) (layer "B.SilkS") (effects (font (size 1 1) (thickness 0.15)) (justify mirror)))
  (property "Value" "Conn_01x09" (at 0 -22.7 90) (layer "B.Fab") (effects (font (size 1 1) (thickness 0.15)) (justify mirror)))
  (pad "1" thru_hole rect (at 0 0 270) (size 1.7 1.7) (drill 1) (layers "*.Cu" "*.Mask") (remove_unused_layers no) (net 9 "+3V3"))
  (pad "2" thru_hole circle (at 0 -2.54 270) (size 1.7 1.7) (drill 1) (layers "*.Cu" "*.Mask") (remove_unused_layers no) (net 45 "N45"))
  (pad "3" thru_hole circle (at 0 -5.08 270) (size 1.7 1.7) (drill 1) (layers "*.Cu" "*.Mask") (remove_unused_layers no) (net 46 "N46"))
  (pad "4" thru_hole circle (at 0 -7.62 270) (size 1.7 1.7) (drill 1) (layers "*.Cu" "*.Mask") (remove_unused_layers no) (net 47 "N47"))
  (pad "5" thru_hole circle (at 0 -10.16 270) (size 1.7 1.7) (drill 1) (layers "*.Cu" "*.Mask") (remove_unused_layers no) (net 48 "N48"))
  (pad "6" thru_hole circle (at 0 -12.7 270) (size 1.7 1.7) (drill 1) (layers "*.Cu" "*.Mask") (remove_unused_layers no) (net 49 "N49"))
  (pad "7" thru_hole circle (at 0 -15.24 270) (size 1.7 1.7) (drill 1) (layers "*.Cu" "*.Mask") (remove_unused_layers no) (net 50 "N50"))
  (pad "8" thru_hole circle (at 0 -17.78 270) (size 1.7 1.7) (drill 1) (layers "*.Cu" "*.Mask") (remove_unused_layers no) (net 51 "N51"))
  (pad "9" thru_hole circle (at 0 -20.32 270) (size 1.7 1.7) (drill 1) (layers "*.Cu" "*.Mask") (remove_unused_layers no) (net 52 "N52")))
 (gr_rect (start 115.6 43.2) (end 162.6 115.2) (stroke (width 0.05) (type default)) (fill no) (layer "Edge.Cuts"))
 (segment (start 127 66.04) (end 124.46 66.04) (width 0.8) (layer "F.Cu") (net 9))
 (via (at 127 66.04) (size 0.6) (drill 0.3) (layers "F.Cu" "B.Cu") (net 9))
 (segment (start 160.02 60.96) (end 160.02 71.12) (width 0.8) (layer "B.Cu") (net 9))
 (segment (start 129.54 71.12) (end 132.08 71.12) (width 0.8) (layer "B.Cu") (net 9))
 (segment (start 142.24 88.9) (end 137.16 88.9) (width 0.8) (layer "B.Cu") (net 9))
 (segment (start 160.02 58.42) (end 160.02 60.96) (width 0.8) (layer "B.Cu") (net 9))
 (segment (start 157.48 88.9) (end 157.48 71.12) (width 0.8) (layer "B.Cu") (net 9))
 (segment (start 129.54 66.04) (end 127 66.04) (width 0.8) (layer "B.Cu") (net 9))
 (segment (start 160.02 71.12) (end 157.48 71.12) (width 0.8) (layer "B.Cu") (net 9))
 (segment (start 137.16 88.9) (end 132.08 88.9) (width 0.8) (layer "B.Cu") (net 9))
 (segment (start 129.54 71.12) (end 129.54 66.04) (width 0.8) (layer "B.Cu") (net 9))
 (segment (start 142.24 88.9) (end 157.48 88.9) (width 0.8) (layer "B.Cu") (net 9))
 (segment (start 132.08 88.9) (end 132.08 93.98) (width 0.8) (layer "B.Cu") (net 9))
 (segment (start 127 68.58) (end 124.46 68.58) (width 0.8) (layer "F.Cu") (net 10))
 (via (at 127 68.58) (size 0.6) (drill 0.3) (layers "F.Cu" "B.Cu") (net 10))
 (segment (start 147.32 68.58) (end 144.78 68.58) (width 0.8) (layer "B.Cu") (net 10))
 (segment (start 129.58 73.66) (end 129.54 73.62) (width 0.8) (layer "B.Cu") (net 10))
 (segment (start 129.54 73.62) (end 127.04 73.62) (width 0.8) (layer "B.Cu") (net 10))
 (segment (start 132.08 73.66) (end 134.62 73.66) (width 0.8) (layer "B.Cu") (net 10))
 (segment (start 144.78 83.82) (end 139.7 83.82) (width 0.8) (layer "B.Cu") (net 10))
 (segment (start 154.94 53.34) (end 147.32 53.34) (width 0.8) (layer "B.Cu") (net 10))
 (segment (start 139.7 78.74) (end 139.7 83.82) (width 0.8) (layer "B.Cu") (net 10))
 (segment (start 127 73.66) (end 127 68.58) (width 0.8) (layer "B.Cu") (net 10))
 (segment (start 144.78 68.58) (end 144.78 83.82) (width 0.8) (layer "B.Cu") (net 10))
 (segment (start 147.32 53.34) (end 147.32 68.58) (width 0.8) (layer "B.Cu") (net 10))
 (segment (start 127.04 73.62) (end 127 73.66) (width 0.8) (layer "B.Cu") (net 10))
 (segment (start 132.08 73.66) (end 129.58 73.66) (width 0.8) (layer "B.Cu") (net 10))
 (segment (start 139.7 78.74) (end 134.62 78.74) (width 0.8) (layer "B.Cu") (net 10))
 (segment (start 134.62 73.66) (end 134.62 78.74) (width 0.8) (layer "B.Cu") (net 10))
 (segment (start 157.44 50.84) (end 157.48 50.8) (width 0.8) (layer "B.Cu") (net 24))
 (segment (start 142.24 53.34) (end 142.24 50.8) (width 0.8) (layer "B.Cu") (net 24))
 (segment (start 142.24 50.8) (end 147.32 50.8) (width 0.8) (layer "B.Cu") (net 24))
 (segment (start 154.9 50.8) (end 154.94 50.84) (width 0.8) (layer "B.Cu") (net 24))
 (segment (start 147.32 50.8) (end 154.9 50.8) (width 0.8) (layer "B.Cu") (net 24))
 (segment (start 139.7 53.34) (end 142.24 53.34) (width 0.8) (layer "B.Cu") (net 24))
 (segment (start 154.94 50.84) (end 157.44 50.84) (width 0.8) (layer "B.Cu") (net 24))
 (segment (start 157.48 58.42) (end 157.48 60.96) (width 0.8) (layer "B.Cu") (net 24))
 (segment (start 157.48 50.8) (end 157.48 58.42) (width 0.8) (layer "B.Cu") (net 24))
 (segment (start 142.24 106.68) (end 127 106.68) (width 0.8) (layer "B.Cu") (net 12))
 (segment (start 142.24 109.22) (end 142.24 106.68) (width 0.8) (layer "B.Cu") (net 12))
 (segment (start 127 78.74) (end 132.08 78.74) (width 0.8) (layer "B.Cu") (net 12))
 (segment (start 127 106.68) (end 127 78.74) (width 0.8) (layer "B.Cu") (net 12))
 (segment (start 129.54 104.14) (end 144.78 104.14) (width 0.8) (layer "B.Cu") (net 13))
 (segment (start 132.08 81.28) (end 129.54 81.28) (width 0.8) (layer "B.Cu") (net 13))
 (segment (start 144.78 104.14) (end 144.78 109.22) (width 0.8) (layer "B.Cu") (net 13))
 (segment (start 129.54 81.28) (end 129.54 104.14) (width 0.8) (layer "B.Cu") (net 13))
 (segment (start 142.24 76.2) (end 142.24 81.28) (width 0.8) (layer "B.Cu") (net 15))
 (segment (start 139.7 76.2) (end 142.24 76.2) (width 0.8) (layer "B.Cu") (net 15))
 (segment (start 152.4 63.5) (end 157.48 63.5) (width 0.8) (layer "B.Cu") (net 34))
 (segment (start 157.48 63.5) (end 157.48 66.12) (width 0.8) (layer "B.Cu") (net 34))
 (segment (start 152.4 66.04) (end 154.94 66.04) (width 0.8) (layer "B.Cu") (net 33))
 (segment (start 154.94 68.58) (end 157.44 68.58) (width 0.8) (layer "B.Cu") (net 33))
 (segment (start 157.44 68.58) (end 157.48 68.62) (width 0.8) (layer "B.Cu") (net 33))
 (segment (start 154.94 66.04) (end 154.94 68.58) (width 0.8) (layer "B.Cu") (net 33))
 (segment (start 144.78 55.88) (end 144.78 63.5) (width 0.8) (layer "B.Cu") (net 23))
 (segment (start 139.7 55.88) (end 144.78 55.88) (width 0.8) (layer "B.Cu") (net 23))
 (segment (start 139.7 58.42) (end 142.24 58.42) (width 0.8) (layer "B.Cu") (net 22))
 (segment (start 142.24 58.42) (end 142.24 66.04) (width 0.8) (layer "B.Cu") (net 22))
 (segment (start 142.24 66.04) (end 144.78 66.04) (width 0.8) (layer "B.Cu") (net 22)))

